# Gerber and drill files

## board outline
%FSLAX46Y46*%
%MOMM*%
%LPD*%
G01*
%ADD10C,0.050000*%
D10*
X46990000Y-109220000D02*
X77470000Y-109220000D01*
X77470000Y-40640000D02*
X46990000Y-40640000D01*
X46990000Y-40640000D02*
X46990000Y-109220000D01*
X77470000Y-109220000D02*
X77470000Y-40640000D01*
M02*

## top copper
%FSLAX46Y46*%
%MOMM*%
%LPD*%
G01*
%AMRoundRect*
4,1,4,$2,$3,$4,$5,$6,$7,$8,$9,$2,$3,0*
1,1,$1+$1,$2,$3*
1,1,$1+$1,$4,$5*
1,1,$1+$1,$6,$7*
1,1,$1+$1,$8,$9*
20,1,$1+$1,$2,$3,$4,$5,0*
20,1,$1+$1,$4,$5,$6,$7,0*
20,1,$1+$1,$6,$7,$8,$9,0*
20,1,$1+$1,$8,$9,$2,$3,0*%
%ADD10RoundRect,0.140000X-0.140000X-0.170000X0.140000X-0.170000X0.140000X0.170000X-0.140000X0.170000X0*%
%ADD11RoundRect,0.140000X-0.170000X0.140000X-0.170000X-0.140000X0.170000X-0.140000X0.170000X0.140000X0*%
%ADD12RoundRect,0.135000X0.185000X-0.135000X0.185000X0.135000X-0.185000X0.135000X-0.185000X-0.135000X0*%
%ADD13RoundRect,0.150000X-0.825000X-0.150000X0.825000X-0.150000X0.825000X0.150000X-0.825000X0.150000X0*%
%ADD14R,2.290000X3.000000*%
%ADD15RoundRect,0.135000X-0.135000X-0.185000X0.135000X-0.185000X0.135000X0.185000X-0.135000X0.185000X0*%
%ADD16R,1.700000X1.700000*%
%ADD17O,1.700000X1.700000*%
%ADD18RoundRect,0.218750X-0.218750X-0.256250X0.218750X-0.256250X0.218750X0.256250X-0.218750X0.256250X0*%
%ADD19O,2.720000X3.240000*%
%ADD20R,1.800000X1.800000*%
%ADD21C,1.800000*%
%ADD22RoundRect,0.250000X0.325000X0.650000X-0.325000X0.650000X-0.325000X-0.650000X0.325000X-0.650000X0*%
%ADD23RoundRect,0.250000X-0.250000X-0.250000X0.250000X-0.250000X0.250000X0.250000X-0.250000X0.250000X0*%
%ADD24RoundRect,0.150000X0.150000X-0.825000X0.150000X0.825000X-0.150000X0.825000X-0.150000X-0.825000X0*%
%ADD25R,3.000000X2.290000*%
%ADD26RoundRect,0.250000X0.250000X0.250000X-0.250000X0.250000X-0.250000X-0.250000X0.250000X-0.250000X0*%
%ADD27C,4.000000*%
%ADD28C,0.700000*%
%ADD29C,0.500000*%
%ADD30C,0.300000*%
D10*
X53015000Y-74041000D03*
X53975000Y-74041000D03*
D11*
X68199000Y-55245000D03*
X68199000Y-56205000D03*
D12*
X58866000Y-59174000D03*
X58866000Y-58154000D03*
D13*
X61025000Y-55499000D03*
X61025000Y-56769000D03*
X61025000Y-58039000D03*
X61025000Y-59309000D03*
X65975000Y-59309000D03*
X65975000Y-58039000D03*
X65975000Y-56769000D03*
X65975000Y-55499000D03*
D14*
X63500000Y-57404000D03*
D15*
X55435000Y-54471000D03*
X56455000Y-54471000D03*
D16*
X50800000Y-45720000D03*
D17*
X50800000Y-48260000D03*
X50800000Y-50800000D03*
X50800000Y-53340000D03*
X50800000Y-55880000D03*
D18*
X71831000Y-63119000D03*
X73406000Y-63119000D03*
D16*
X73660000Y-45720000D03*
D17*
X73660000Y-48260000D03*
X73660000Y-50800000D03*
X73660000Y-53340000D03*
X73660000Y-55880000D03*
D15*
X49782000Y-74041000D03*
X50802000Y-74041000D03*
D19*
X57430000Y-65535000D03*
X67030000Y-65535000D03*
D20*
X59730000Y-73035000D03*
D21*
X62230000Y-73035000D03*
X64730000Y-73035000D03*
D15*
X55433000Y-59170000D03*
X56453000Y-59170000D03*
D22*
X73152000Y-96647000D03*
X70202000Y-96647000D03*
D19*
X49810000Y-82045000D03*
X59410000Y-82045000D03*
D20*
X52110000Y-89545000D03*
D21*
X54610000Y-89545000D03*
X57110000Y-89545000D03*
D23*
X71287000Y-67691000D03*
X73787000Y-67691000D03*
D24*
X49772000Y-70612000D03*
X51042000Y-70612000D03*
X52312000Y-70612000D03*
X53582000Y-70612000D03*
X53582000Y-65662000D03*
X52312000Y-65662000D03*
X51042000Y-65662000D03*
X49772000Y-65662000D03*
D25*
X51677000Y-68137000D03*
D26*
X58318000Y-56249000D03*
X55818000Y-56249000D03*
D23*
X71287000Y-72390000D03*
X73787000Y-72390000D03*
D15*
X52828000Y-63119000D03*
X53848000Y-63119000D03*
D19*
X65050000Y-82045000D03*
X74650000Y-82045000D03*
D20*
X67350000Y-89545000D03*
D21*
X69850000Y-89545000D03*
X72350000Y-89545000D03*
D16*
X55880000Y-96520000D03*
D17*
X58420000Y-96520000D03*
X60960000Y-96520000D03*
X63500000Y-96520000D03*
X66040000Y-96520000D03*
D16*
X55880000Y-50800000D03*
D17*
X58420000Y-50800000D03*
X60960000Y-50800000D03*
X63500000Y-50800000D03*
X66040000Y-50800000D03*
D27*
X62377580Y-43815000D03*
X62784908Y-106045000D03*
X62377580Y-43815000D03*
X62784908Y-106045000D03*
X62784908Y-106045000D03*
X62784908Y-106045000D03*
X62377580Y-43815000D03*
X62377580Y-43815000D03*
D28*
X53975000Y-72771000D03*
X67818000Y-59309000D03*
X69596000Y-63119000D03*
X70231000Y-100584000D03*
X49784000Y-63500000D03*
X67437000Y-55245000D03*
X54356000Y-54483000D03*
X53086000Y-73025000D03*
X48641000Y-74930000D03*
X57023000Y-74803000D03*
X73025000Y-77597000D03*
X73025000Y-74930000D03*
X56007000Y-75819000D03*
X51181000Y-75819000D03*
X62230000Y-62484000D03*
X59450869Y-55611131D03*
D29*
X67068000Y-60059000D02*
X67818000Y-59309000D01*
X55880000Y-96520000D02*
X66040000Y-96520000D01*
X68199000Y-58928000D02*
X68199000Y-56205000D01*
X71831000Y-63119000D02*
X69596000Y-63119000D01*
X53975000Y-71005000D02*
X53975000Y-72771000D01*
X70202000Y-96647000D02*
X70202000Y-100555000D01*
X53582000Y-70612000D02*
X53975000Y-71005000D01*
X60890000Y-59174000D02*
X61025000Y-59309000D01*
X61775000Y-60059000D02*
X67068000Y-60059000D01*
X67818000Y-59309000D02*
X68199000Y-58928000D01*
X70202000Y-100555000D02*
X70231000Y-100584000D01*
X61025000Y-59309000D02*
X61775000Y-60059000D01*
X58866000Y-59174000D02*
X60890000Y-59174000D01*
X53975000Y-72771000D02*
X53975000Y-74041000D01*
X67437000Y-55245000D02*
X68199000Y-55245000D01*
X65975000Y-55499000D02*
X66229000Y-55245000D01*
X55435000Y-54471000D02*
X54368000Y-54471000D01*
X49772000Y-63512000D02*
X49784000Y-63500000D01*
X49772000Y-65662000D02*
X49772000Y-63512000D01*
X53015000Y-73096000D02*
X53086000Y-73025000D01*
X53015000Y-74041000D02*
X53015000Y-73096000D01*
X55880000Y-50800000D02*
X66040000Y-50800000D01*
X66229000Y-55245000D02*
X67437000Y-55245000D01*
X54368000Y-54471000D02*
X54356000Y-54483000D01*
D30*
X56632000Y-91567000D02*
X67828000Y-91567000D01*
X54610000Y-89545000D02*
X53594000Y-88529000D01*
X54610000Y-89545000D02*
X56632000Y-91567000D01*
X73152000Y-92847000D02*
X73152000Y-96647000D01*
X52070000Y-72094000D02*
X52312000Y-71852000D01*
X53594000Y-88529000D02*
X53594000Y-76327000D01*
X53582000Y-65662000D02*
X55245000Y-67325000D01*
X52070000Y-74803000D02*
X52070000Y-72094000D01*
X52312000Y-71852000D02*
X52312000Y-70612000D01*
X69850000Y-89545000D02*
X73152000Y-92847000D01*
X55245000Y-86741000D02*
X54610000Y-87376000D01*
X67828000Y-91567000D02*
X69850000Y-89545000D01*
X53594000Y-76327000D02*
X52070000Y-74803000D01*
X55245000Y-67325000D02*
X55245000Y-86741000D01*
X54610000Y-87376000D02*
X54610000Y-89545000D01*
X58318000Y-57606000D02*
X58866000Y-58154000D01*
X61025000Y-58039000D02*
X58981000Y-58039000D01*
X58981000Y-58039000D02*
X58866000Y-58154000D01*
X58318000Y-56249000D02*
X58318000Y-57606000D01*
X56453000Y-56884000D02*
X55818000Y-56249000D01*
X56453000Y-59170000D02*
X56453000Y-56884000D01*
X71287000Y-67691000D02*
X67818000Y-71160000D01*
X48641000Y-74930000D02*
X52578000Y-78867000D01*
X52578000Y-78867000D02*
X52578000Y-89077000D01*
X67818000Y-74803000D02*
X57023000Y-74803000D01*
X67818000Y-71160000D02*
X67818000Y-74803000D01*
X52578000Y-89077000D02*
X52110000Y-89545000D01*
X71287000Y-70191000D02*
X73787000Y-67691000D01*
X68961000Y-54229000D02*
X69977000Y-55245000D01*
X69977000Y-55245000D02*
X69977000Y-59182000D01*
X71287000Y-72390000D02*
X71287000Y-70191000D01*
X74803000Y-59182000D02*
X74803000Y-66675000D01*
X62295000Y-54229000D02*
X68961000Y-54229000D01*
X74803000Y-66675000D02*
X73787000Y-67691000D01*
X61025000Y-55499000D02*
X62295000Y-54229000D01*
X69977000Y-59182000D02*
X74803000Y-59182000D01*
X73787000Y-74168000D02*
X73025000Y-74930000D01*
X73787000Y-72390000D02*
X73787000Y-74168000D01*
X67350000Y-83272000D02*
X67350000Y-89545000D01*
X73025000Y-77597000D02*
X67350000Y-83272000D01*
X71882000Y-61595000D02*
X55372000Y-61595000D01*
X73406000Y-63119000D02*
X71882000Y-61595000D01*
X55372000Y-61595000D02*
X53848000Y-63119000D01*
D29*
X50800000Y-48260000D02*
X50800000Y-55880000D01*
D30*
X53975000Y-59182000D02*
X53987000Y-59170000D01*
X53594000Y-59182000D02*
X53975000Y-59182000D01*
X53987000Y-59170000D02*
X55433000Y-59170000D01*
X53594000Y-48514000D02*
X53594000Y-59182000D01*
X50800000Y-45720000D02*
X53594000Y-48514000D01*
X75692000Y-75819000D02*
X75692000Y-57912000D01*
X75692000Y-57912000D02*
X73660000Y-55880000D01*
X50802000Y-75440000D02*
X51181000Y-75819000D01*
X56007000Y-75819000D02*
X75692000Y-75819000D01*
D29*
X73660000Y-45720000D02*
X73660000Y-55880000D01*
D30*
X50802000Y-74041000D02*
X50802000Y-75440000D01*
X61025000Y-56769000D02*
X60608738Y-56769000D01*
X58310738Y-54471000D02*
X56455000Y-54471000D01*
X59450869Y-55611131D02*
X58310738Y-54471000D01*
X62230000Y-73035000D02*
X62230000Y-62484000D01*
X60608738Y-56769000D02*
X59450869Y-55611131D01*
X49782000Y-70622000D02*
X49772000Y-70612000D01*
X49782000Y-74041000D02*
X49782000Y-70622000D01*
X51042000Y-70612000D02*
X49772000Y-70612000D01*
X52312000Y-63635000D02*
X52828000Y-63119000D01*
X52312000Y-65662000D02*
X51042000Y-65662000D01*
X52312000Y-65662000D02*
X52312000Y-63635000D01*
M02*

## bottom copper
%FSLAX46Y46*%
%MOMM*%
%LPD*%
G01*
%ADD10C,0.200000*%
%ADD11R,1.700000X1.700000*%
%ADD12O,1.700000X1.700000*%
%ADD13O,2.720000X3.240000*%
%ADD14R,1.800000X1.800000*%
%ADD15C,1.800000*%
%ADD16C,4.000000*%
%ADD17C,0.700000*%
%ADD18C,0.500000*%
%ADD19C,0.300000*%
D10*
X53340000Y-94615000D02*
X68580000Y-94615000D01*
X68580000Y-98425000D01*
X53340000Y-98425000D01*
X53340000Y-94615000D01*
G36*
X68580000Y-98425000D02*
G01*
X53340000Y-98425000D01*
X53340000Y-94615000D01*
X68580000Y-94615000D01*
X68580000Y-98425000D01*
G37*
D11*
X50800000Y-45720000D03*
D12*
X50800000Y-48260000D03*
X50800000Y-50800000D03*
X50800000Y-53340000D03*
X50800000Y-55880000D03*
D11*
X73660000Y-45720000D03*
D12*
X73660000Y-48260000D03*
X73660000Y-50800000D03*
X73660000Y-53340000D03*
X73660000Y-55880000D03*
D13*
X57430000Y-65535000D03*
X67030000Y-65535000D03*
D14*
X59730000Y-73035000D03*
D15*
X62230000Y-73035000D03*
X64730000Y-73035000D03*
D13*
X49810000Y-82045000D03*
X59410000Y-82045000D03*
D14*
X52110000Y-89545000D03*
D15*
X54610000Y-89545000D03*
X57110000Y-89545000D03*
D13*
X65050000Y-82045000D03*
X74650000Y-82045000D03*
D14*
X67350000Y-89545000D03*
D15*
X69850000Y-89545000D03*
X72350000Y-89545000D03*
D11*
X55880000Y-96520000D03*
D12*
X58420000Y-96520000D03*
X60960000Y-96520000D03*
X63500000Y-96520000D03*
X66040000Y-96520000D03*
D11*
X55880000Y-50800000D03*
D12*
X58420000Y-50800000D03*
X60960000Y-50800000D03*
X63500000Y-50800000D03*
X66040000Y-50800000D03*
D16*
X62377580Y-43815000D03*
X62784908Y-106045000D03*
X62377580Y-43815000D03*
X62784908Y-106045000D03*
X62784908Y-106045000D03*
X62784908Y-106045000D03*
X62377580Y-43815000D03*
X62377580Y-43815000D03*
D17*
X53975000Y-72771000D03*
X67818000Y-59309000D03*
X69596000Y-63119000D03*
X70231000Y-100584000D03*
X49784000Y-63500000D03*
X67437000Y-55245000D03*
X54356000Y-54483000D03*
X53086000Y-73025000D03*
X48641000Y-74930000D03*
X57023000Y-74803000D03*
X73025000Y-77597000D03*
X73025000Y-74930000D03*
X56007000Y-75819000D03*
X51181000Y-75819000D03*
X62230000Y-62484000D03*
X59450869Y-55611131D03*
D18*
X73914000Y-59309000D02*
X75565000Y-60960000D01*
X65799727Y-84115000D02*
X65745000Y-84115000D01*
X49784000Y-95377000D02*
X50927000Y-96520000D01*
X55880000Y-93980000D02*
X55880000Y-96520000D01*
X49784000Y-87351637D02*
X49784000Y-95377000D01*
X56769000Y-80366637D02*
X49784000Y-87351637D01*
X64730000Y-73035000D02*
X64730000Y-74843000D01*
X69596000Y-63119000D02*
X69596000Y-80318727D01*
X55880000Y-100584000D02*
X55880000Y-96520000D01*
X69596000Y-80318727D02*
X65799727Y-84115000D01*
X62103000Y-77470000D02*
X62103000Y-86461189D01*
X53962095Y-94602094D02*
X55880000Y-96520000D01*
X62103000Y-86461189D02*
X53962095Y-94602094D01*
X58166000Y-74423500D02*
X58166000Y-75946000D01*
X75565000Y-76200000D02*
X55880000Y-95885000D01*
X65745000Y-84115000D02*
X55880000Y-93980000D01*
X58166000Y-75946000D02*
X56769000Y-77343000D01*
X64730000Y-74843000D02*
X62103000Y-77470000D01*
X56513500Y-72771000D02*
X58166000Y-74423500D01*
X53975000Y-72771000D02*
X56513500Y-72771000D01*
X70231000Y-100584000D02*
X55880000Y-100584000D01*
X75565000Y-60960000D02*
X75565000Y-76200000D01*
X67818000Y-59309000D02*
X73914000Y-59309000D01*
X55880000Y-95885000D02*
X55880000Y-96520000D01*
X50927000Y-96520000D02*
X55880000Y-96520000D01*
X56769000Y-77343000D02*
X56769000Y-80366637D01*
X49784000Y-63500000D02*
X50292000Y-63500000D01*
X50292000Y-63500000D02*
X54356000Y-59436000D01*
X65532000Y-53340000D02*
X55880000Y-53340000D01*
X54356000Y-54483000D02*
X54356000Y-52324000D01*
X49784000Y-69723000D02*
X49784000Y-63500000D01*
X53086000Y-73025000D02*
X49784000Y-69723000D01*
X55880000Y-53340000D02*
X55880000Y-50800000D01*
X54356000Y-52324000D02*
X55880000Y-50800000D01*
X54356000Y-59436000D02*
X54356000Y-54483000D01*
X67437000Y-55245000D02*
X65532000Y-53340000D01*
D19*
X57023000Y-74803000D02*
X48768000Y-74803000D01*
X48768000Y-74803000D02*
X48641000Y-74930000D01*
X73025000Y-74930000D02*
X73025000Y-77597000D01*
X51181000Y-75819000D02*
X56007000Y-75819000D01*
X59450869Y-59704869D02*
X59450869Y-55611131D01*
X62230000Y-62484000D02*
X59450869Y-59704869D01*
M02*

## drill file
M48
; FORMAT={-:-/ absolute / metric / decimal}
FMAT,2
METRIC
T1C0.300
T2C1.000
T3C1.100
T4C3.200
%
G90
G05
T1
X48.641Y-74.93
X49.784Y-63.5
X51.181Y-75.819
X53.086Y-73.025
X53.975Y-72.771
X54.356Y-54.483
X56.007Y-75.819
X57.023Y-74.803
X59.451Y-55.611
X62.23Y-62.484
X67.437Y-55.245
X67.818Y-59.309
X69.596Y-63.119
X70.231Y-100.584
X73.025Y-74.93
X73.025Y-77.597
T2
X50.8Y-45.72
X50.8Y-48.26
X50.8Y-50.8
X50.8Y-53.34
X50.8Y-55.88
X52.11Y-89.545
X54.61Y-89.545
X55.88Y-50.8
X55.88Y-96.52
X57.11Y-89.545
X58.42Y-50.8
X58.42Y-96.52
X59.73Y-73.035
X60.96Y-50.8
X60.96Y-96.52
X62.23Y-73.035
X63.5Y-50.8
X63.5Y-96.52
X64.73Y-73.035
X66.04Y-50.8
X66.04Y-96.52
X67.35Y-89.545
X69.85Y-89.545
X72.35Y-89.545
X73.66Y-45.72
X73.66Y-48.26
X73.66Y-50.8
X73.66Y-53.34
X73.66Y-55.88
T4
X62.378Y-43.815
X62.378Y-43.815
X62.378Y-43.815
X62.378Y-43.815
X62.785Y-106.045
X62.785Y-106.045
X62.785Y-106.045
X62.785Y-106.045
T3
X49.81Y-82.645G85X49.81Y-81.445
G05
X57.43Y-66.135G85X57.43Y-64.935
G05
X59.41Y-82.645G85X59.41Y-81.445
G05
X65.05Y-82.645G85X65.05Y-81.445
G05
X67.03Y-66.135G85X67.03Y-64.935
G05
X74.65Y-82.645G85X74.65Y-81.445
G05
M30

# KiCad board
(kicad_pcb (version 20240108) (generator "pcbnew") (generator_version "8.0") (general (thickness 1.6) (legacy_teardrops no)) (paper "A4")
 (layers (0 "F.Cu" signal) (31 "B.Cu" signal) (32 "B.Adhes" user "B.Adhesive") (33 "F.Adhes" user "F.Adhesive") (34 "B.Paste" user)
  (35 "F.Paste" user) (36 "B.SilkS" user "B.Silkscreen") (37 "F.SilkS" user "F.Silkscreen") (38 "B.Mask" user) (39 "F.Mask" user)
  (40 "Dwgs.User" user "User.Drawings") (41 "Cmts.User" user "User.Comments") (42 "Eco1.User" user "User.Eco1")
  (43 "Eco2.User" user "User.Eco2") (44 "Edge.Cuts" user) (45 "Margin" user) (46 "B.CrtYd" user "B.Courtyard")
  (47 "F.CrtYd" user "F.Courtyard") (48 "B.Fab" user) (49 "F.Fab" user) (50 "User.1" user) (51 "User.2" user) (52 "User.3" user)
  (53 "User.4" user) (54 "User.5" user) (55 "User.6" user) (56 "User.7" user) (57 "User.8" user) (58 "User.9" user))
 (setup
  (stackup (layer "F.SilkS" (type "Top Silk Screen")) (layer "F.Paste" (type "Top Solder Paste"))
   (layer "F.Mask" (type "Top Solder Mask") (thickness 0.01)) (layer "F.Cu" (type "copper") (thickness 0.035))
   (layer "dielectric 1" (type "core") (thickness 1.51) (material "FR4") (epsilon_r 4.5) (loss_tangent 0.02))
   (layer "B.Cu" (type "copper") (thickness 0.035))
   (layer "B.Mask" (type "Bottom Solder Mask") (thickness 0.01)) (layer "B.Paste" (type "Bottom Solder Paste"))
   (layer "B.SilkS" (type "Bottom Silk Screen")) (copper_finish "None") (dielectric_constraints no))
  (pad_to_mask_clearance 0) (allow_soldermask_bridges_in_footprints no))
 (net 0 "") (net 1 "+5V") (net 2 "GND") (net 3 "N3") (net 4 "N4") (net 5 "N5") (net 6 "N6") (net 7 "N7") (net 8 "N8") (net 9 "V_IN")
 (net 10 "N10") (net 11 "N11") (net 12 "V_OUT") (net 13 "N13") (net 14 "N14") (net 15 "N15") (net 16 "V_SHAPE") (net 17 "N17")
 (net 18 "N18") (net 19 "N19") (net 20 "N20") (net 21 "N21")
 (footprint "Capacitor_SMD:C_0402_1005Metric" (layer "F.Cu") (at 53.495 74.041)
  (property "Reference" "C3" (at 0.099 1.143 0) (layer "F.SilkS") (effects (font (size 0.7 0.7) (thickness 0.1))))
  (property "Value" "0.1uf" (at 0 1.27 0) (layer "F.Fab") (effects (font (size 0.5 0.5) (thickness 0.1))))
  (pad "1" smd roundrect (at -0.48 0) (size 0.56 0.62) (layers "F.Cu" "F.Paste" "F.Mask") (roundrect_rratio 0.25) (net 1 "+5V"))
  (pad "2" smd roundrect (at 0.48 0) (size 0.56 0.62) (layers "F.Cu" "F.Paste" "F.Mask") (roundrect_rratio 0.25) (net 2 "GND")))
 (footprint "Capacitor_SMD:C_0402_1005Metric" (layer "F.Cu") (at 68.199 55.725 -90)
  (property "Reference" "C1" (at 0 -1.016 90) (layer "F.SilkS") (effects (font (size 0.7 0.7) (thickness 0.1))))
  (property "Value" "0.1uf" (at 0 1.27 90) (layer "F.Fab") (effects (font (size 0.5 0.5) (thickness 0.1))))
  (pad "1" smd roundrect (at -0.48 0 270) (size 0.56 0.62) (layers "F.Cu" "F.Paste" "F.Mask") (roundrect_rratio 0.25) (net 1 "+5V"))
  (pad "2" smd roundrect (at 0.48 0 270) (size 0.56 0.62) (layers "F.Cu" "F.Paste" "F.Mask") (roundrect_rratio 0.25) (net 2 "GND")))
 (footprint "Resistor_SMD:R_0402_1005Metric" (layer "F.Cu") (at 58.866 58.664 90)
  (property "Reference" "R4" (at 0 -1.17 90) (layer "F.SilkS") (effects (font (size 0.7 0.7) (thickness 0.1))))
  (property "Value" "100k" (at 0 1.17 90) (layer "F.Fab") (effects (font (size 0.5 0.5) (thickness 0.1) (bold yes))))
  (pad "1" smd roundrect (at -0.51 0 90) (size 0.54 0.64) (layers "F.Cu" "F.Paste" "F.Mask") (roundrect_rratio 0.25) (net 2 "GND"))
  (pad "2" smd roundrect (at 0.51 0 90) (size 0.54 0.64) (layers "F.Cu" "F.Paste" "F.Mask") (roundrect_rratio 0.25) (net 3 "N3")))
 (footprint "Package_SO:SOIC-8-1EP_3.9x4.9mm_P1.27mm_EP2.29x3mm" (layer "F.Cu") (at 63.5 57.404)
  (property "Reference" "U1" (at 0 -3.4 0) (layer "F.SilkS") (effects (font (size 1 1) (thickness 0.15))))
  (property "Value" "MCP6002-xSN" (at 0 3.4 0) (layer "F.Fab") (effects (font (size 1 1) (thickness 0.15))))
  (pad "" smd roundrect (at -0.57 -0.75) (size 0.92 1.21) (layers "F.Paste") (roundrect_rratio 0.25))
  (pad "" smd roundrect (at -0.57 0.75) (size 0.92 1.21) (layers "F.Paste") (roundrect_rratio 0.25))
  (pad "" smd roundrect (at 0.57 -0.75) (size 0.92 1.21) (layers "F.Paste") (roundrect_rratio 0.25))
  (pad "" smd roundrect (at 0.57 0.75) (size 0.92 1.21) (layers "F.Paste") (roundrect_rratio 0.25))
  (pad "1" smd roundrect (at -2.475 -1.905) (size 1.95 0.6) (layers "F.Cu" "F.Paste" "F.Mask") (roundrect_rratio 0.25) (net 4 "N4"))
  (pad "2" smd roundrect (at -2.475 -0.635) (size 1.95 0.6) (layers "F.Cu" "F.Paste" "F.Mask") (roundrect_rratio 0.25) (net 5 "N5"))
  (pad "3" smd roundrect (at -2.475 0.635) (size 1.95 0.6) (layers "F.Cu" "F.Paste" "F.Mask") (roundrect_rratio 0.25) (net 3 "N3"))
  (pad "4" smd roundrect (at -2.475 1.905) (size 1.95 0.6) (layers "F.Cu" "F.Paste" "F.Mask") (roundrect_rratio 0.25) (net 2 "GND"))
  (pad "5" smd roundrect (at 2.475 1.905) (size 1.95 0.6) (layers "F.Cu" "F.Paste" "F.Mask") (roundrect_rratio 0.25) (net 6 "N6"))
  (pad "6" smd roundrect (at 2.475 0.635) (size 1.95 0.6) (layers "F.Cu" "F.Paste" "F.Mask") (roundrect_rratio 0.25) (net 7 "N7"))
  (pad "7" smd roundrect (at 2.475 -0.635) (size 1.95 0.6) (layers "F.Cu" "F.Paste" "F.Mask") (roundrect_rratio 0.25) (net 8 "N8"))
  (pad "8" smd roundrect (at 2.475 -1.905) (size 1.95 0.6) (layers "F.Cu" "F.Paste" "F.Mask") (roundrect_rratio 0.25) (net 1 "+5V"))
  (pad "9" smd rect (at 0 0) (size 2.29 3) (layers "F.Cu" "F.Mask") (zone_connect 2)))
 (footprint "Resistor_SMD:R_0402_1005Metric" (layer "F.Cu") (at 55.945 54.471)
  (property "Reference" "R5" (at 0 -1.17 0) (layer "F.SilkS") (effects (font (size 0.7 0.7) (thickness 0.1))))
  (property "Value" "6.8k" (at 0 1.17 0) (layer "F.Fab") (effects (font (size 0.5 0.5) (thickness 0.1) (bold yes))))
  (pad "1" smd roundrect (at -0.51 0) (size 0.54 0.64) (layers "F.Cu" "F.Paste" "F.Mask") (roundrect_rratio 0.25) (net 1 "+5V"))
  (pad "2" smd roundrect (at 0.51 0) (size 0.54 0.64) (layers "F.Cu" "F.Paste" "F.Mask") (roundrect_rratio 0.25) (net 5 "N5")))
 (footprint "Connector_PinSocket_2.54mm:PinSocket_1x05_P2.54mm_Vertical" (layer "F.Cu") (at 50.8 45.72)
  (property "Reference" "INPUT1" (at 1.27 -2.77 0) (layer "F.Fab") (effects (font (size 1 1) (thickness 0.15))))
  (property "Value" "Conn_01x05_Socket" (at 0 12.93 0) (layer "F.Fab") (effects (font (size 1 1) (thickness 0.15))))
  (pad "1" thru_hole rect (at 0 0) (size 1.7 1.7) (drill 1) (layers "*.Cu" "*.Mask") (remove_unused_layers no) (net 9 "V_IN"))
  (pad "2" thru_hole oval (at 0 2.54) (size 1.7 1.7) (drill 1) (layers "*.Cu" "*.Mask") (remove_unused_layers no) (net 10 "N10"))
  (pad "3" thru_hole oval (at 0 5.08) (size 1.7 1.7) (drill 1) (layers "*.Cu" "*.Mask") (remove_unused_layers no) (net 10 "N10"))
  (pad "4" thru_hole oval (at 0 7.62) (size 1.7 1.7) (drill 1) (layers "*.Cu" "*.Mask") (remove_unused_layers no) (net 10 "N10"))
  (pad "5" thru_hole oval (at 0 10.16) (size 1.7 1.7) (drill 1) (layers "*.Cu" "*.Mask") (remove_unused_layers no) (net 10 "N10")))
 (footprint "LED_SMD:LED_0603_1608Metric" (layer "F.Cu") (at 72.6185 63.119)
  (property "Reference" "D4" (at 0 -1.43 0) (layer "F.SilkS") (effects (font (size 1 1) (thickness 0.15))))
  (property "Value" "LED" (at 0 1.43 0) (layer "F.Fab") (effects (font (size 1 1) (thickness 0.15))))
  (pad "1" smd roundrect (at -0.7875 0) (size 0.875 0.95) (layers "F.Cu" "F.Paste" "F.Mask") (roundrect_rratio 0.25) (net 2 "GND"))
  (pad "2" smd roundrect (at 0.7875 0) (size 0.875 0.95) (layers "F.Cu" "F.Paste" "F.Mask") (roundrect_rratio 0.25) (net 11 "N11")))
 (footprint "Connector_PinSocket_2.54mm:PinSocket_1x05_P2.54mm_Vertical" (layer "F.Cu") (at 73.66 45.72)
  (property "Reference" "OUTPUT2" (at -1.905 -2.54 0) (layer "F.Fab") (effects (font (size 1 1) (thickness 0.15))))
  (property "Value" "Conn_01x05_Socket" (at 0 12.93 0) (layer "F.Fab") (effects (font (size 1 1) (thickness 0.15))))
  (pad "1" thru_hole rect (at 0 0) (size 1.7 1.7) (drill 1) (layers "*.Cu" "*.Mask") (remove_unused_layers no) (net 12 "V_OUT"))
  (pad "2" thru_hole oval (at 0 2.54) (size 1.7 1.7) (drill 1) (layers "*.Cu" "*.Mask") (remove_unused_layers no) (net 12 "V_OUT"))
  (pad "3" thru_hole oval (at 0 5.08) (size 1.7 1.7) (drill 1) (layers "*.Cu" "*.Mask") (remove_unused_layers no) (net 12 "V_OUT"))
  (pad "4" thru_hole oval (at 0 7.62) (size 1.7 1.7) (drill 1) (layers "*.Cu" "*.Mask") (remove_unused_layers no) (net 12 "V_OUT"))
  (pad "5" thru_hole oval (at 0 10.16) (size 1.7 1.7) (drill 1) (layers "*.Cu" "*.Mask") (remove_unused_layers no) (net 12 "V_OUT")))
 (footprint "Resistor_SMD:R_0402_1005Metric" (layer "F.Cu") (at 50.292 74.041)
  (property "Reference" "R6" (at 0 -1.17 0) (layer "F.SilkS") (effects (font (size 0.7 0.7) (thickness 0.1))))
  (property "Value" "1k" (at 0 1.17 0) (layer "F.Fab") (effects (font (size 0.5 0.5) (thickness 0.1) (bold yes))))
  (pad "1" smd roundrect (at -0.51 0) (size 0.54 0.64) (layers "F.Cu" "F.Paste" "F.Mask") (roundrect_rratio 0.25) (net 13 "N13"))
  (pad "2" smd roundrect (at 0.51 0) (size 0.54 0.64) (layers "F.Cu" "F.Paste" "F.Mask") (roundrect_rratio 0.25) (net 12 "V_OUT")))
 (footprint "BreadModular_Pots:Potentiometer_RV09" (layer "F.Cu") (at 59.73 73.035 90)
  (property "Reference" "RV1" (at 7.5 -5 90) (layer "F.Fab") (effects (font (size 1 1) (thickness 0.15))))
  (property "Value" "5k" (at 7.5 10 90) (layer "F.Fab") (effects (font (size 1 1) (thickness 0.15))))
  (pad "" thru_hole oval (at 7.5 -2.3 180) (size 2.72 3.24) (drill oval 1.1 2.3) (layers "*.Cu" "*.Mask") (remove_unused_layers no))
  (pad "" thru_hole oval (at 7.5 7.3 180) (size 2.72 3.24) (drill oval 1.1 2.3) (layers "*.Cu" "*.Mask") (remove_unused_layers no))
  (pad "1" thru_hole rect (at 0 0 180) (size 1.8 1.8) (drill 1) (layers "*.Cu" "*.Mask") (remove_unused_layers no) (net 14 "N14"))
  (pad "2" thru_hole circle (at 0 2.5 180) (size 1.8 1.8) (drill 1) (layers "*.Cu" "*.Mask") (remove_unused_layers no) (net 5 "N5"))
  (pad "3" thru_hole circle (at 0 5 180) (size 1.8 1.8) (drill 1) (layers "*.Cu" "*.Mask") (remove_unused_layers no) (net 2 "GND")))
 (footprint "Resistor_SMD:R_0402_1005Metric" (layer "F.Cu") (at 55.943 59.17)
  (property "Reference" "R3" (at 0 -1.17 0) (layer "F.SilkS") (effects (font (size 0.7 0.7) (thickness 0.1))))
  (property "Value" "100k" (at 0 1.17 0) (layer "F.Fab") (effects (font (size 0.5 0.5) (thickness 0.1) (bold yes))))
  (pad "1" smd roundrect (at -0.51 0) (size 0.54 0.64) (layers "F.Cu" "F.Paste" "F.Mask") (roundrect_rratio 0.25) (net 9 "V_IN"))
  (pad "2" smd roundrect (at 0.51 0) (size 0.54 0.64) (layers "F.Cu" "F.Paste" "F.Mask") (roundrect_rratio 0.25) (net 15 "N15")))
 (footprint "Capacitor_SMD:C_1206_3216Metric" (layer "F.Cu") (at 71.677 96.647 180)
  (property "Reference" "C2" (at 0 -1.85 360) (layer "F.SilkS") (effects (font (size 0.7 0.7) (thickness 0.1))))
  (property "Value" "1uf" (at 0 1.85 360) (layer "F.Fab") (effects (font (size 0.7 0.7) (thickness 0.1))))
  (pad "1" smd roundrect (at -1.475 0 180) (size 1.15 1.8) (layers "F.Cu" "F.Paste" "F.Mask") (roundrect_rratio 0.217391) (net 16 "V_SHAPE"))
  (pad "2" smd roundrect (at 1.475 0 180) (size 1.15 1.8) (layers "F.Cu" "F.Paste" "F.Mask") (roundrect_rratio 0.217391) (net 2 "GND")))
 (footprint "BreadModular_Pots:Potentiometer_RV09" (layer "F.Cu") (at 52.11 89.545 90)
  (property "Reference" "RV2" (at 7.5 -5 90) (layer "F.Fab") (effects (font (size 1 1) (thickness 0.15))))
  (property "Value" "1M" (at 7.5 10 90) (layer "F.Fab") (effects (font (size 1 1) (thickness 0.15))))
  (pad "" thru_hole oval (at 7.5 -2.3 180) (size 2.72 3.24) (drill oval 1.1 2.3) (layers "*.Cu" "*.Mask") (remove_unused_layers no))
  (pad "" thru_hole oval (at 7.5 7.3 180) (size 2.72 3.24) (drill oval 1.1 2.3) (layers "*.Cu" "*.Mask") (remove_unused_layers no))
  (pad "1" thru_hole rect (at 0 0 180) (size 1.8 1.8) (drill 1) (layers "*.Cu" "*.Mask") (remove_unused_layers no) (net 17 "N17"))
  (pad "2" thru_hole circle (at 0 2.5 180) (size 1.8 1.8) (drill 1) (layers "*.Cu" "*.Mask") (remove_unused_layers no) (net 16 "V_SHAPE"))
  (pad "3" thru_hole circle (at 0 5 180) (size 1.8 1.8) (drill 1) (layers "*.Cu" "*.Mask") (remove_unused_layers no) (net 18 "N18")))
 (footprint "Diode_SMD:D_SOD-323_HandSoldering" (layer "F.Cu") (at 72.537 67.691)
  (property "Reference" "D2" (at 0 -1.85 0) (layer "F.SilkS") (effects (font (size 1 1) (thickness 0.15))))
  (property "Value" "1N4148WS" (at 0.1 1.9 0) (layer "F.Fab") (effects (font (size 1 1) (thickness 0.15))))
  (pad "1" smd roundrect (at -1.25 0) (size 1 1) (layers "F.Cu" "F.Paste" "F.Mask") (roundrect_rratio 0.25) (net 17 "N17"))
  (pad "2" smd roundrect (at 1.25 0) (size 1 1) (layers "F.Cu" "F.Paste" "F.Mask") (roundrect_rratio 0.25) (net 4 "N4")))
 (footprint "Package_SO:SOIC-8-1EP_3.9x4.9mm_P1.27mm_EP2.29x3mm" (layer "F.Cu") (at 51.677 68.137 90)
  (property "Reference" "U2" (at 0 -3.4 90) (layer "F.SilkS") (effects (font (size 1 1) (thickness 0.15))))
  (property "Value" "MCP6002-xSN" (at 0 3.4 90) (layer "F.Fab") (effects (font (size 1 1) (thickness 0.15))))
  (pad "" smd roundrect (at -0.57 -0.75 90) (size 0.92 1.21) (layers "F.Paste") (roundrect_rratio 0.25))
  (pad "" smd roundrect (at -0.57 0.75 90) (size 0.92 1.21) (layers "F.Paste") (roundrect_rratio 0.25))
  (pad "" smd roundrect (at 0.57 -0.75 90) (size 0.92 1.21) (layers "F.Paste") (roundrect_rratio 0.25))
  (pad "" smd roundrect (at 0.57 0.75 90) (size 0.92 1.21) (layers "F.Paste") (roundrect_rratio 0.25))
  (pad "1" smd roundrect (at -2.475 -1.905 90) (size 1.95 0.6) (layers "F.Cu" "F.Paste" "F.Mask") (roundrect_rratio 0.25) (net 13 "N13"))
  (pad "2" smd roundrect (at -2.475 -0.635 90) (size 1.95 0.6) (layers "F.Cu" "F.Paste" "F.Mask") (roundrect_rratio 0.25) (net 13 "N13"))
  (pad "3" smd roundrect (at -2.475 0.635 90) (size 1.95 0.6) (layers "F.Cu" "F.Paste" "F.Mask") (roundrect_rratio 0.25) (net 16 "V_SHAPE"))
  (pad "4" smd roundrect (at -2.475 1.905 90) (size 1.95 0.6) (layers "F.Cu" "F.Paste" "F.Mask") (roundrect_rratio 0.25) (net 2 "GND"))
  (pad "5" smd roundrect (at 2.475 1.905 90) (size 1.95 0.6) (layers "F.Cu" "F.Paste" "F.Mask") (roundrect_rratio 0.25) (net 16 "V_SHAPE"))
  (pad "6" smd roundrect (at 2.475 0.635 90) (size 1.95 0.6) (layers "F.Cu" "F.Paste" "F.Mask") (roundrect_rratio 0.25) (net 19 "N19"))
  (pad "7" smd roundrect (at 2.475 -0.635 90) (size 1.95 0.6) (layers "F.Cu" "F.Paste" "F.Mask") (roundrect_rratio 0.25) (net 19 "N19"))
  (pad "8" smd roundrect (at 2.475 -1.905 90) (size 1.95 0.6) (layers "F.Cu" "F.Paste" "F.Mask") (roundrect_rratio 0.25) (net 1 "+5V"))
  (pad "9" smd rect (at 0 0 90) (size 2.29 3) (layers "F.Cu" "F.Mask") (zone_connect 2)))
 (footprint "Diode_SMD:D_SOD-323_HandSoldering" (layer "F.Cu") (at 57.068 56.249 180)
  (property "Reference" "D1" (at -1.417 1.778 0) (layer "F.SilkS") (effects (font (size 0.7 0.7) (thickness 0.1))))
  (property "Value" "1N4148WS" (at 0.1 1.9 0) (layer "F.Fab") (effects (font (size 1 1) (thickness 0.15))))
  (pad "1" smd roundrect (at -1.25 0 180) (size 1 1) (layers "F.Cu" "F.Paste" "F.Mask") (roundrect_rratio 0.25) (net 3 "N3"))
  (pad "2" smd roundrect (at 1.25 0 180) (size 1 1) (layers "F.Cu" "F.Paste" "F.Mask") (roundrect_rratio 0.25) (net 15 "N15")))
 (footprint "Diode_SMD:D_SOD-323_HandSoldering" (layer "F.Cu") (at 72.537 72.39)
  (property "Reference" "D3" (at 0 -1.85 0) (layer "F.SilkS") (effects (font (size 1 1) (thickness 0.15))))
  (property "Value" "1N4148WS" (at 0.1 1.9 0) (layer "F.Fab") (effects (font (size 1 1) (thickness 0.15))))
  (pad "1" smd roundrect (at -1.25 0) (size 1 1) (layers "F.Cu" "F.Paste" "F.Mask") (roundrect_rratio 0.25) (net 4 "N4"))
  (pad "2" smd roundrect (at 1.25 0) (size 1 1) (layers "F.Cu" "F.Paste" "F.Mask") (roundrect_rratio 0.25) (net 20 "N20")))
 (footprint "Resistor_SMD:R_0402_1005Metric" (layer "F.Cu") (at 53.338 63.119)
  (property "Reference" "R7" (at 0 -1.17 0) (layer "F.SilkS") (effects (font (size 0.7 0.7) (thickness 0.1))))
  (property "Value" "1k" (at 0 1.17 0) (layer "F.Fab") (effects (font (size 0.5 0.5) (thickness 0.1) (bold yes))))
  (pad "1" smd roundrect (at -0.51 0) (size 0.54 0.64) (layers "F.Cu" "F.Paste" "F.Mask") (roundrect_rratio 0.25) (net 19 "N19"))
  (pad "2" smd roundrect (at 0.51 0) (size 0.54 0.64) (layers "F.Cu" "F.Paste" "F.Mask") (roundrect_rratio 0.25) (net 11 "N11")))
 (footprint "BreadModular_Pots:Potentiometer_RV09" (layer "F.Cu") (at 67.35 89.545 90)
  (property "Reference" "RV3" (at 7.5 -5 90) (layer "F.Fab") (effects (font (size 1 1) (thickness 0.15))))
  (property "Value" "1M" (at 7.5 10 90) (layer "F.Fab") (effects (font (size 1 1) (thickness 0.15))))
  (pad "" thru_hole oval (at 7.5 -2.3 180) (size 2.72 3.24) (drill oval 1.1 2.3) (layers "*.Cu" "*.Mask") (remove_unused_layers no))
  (pad "" thru_hole oval (at 7.5 7.3 180) (size 2.72 3.24) (drill oval 1.1 2.3) (layers "*.Cu" "*.Mask") (remove_unused_layers no))
  (pad "1" thru_hole rect (at 0 0 180) (size 1.8 1.8) (drill 1) (layers "*.Cu" "*.Mask") (remove_unused_layers no) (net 20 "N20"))
  (pad "2" thru_hole circle (at 0 2.5 180) (size 1.8 1.8) (drill 1) (layers "*.Cu" "*.Mask") (remove_unused_layers no) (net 16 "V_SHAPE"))
  (pad "3" thru_hole circle (at 0 5 180) (size 1.8 1.8) (drill 1) (layers "*.Cu" "*.Mask") (remove_unused_layers no) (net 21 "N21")))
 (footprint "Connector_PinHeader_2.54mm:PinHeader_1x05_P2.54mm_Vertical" (layer "B.Cu") (at 55.88 96.52 -90)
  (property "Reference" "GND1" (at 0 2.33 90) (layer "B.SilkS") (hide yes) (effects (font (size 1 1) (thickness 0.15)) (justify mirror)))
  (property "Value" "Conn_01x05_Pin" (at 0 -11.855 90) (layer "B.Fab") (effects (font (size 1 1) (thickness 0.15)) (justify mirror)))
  (pad "1" thru_hole rect (at 0 0 270) (size 1.7 1.7) (drill 1) (layers "*.Cu" "*.Mask") (remove_unused_layers no) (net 2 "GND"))
  (pad "2" thru_hole oval (at 0 -2.54 270) (size 1.7 1.7) (drill 1) (layers "*.Cu" "*.Mask") (remove_unused_layers no) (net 2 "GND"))
  (pad "3" thru_hole oval (at 0 -5.08 270) (size 1.7 1.7) (drill 1) (layers "*.Cu" "*.Mask") (remove_unused_layers no) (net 2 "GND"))
  (pad "4" thru_hole oval (at 0 -7.62 270) (size 1.7 1.7) (drill 1) (layers "*.Cu" "*.Mask") (remove_unused_layers no) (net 2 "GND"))
  (pad "5" thru_hole oval (at 0 -10.16 270) (size 1.7 1.7) (drill 1) (layers "*.Cu" "*.Mask") (remove_unused_layers no) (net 2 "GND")))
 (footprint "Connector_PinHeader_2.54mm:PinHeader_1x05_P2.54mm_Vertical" (layer "B.Cu") (at 55.88 50.8 -90)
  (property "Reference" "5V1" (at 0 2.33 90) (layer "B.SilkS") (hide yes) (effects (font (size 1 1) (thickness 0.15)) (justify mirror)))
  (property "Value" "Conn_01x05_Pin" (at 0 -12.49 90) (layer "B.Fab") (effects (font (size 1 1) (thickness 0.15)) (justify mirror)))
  (pad "1" thru_hole rect (at 0 0 270) (size 1.7 1.7) (drill 1) (layers "*.Cu" "*.Mask") (remove_unused_layers no) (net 1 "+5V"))
  (pad "2" thru_hole oval (at 0 -2.54 270) (size 1.7 1.7) (drill 1) (layers "*.Cu" "*.Mask") (remove_unused_layers no) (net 1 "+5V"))
  (pad "3" thru_hole oval (at 0 -5.08 270) (size 1.7 1.7) (drill 1) (layers "*.Cu" "*.Mask") (remove_unused_layers no) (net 1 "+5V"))
  (pad "4" thru_hole oval (at 0 -7.62 270) (size 1.7 1.7) (drill 1) (layers "*.Cu" "*.Mask") (remove_unused_layers no) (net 1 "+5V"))
  (pad "5" thru_hole oval (at 0 -10.16 270) (size 1.7 1.7) (drill 1) (layers "*.Cu" "*.Mask") (remove_unused_layers no) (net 1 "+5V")))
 (gr_poly
  (pts (xy 53.34 94.615) (xy 68.58 94.615) (xy 68.58 98.425) (xy 53.34 98.425)) (stroke (width 0.2) (type solid)) (fill solid)
  (layer "B.Cu") (net 2))
 (gr_line (start 46.99 109.22) (end 77.47 109.22) (stroke (width 0.05) (type default)) (layer "Edge.Cuts"))
 (gr_line (start 77.47 40.64) (end 46.99 40.64) (stroke (width 0.05) (type default)) (layer "Edge.Cuts"))
 (gr_line (start 46.99 40.64) (end 46.99 109.22) (stroke (width 0.05) (type default)) (layer "Edge.Cuts"))
 (gr_line (start 77.47 109.22) (end 77.47 40.64) (stroke (width 0.05) (type default)) (layer "Edge.Cuts"))
 (via (at 62.37758 43.815) (size 4) (drill 3.2) (layers "F.Cu" "B.Cu") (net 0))
 (via (at 62.784908 106.045) (size 4) (drill 3.2) (layers "F.Cu" "B.Cu") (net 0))
 (via (at 62.37758 43.815) (size 4) (drill 3.2) (layers "F.Cu" "B.Cu") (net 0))
 (via (at 62.784908 106.045) (size 4) (drill 3.2) (layers "F.Cu" "B.Cu") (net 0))
 (via (at 62.784908 106.045) (size 4) (drill 3.2) (layers "F.Cu" "B.Cu") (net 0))
 (via (at 62.784908 106.045) (size 4) (drill 3.2) (layers "F.Cu" "B.Cu") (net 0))
 (via (at 62.37758 43.815) (size 4) (drill 3.2) (layers "F.Cu" "B.Cu") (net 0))
 (via (at 62.37758 43.815) (size 4) (drill 3.2) (layers "F.Cu" "B.Cu") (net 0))
 (segment (start 67.068 60.059) (end 67.818 59.309) (width 0.5) (layer "F.Cu") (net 2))
 (segment (start 55.88 96.52) (end 66.04 96.52) (width 0.5) (layer "F.Cu") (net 2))
 (segment (start 68.199 58.928) (end 68.199 56.205) (width 0.5) (layer "F.Cu") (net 2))
 (segment (start 71.831 63.119) (end 69.596 63.119) (width 0.5) (layer "F.Cu") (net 2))
 (segment (start 53.975 71.005) (end 53.975 72.771) (width 0.5) (layer "F.Cu") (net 2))
 (segment (start 70.202 96.647) (end 70.202 100.555) (width 0.5) (layer "F.Cu") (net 2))
 (segment (start 53.582 70.612) (end 53.975 71.005) (width 0.5) (layer "F.Cu") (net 2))
 (segment (start 60.89 59.174) (end 61.025 59.309) (width 0.5) (layer "F.Cu") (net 2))
 (segment (start 61.775 60.059) (end 67.068 60.059) (width 0.5) (layer "F.Cu") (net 2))
 (segment (start 67.818 59.309) (end 68.199 58.928) (width 0.5) (layer "F.Cu") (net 2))
 (segment (start 70.202 100.555) (end 70.231 100.584) (width 0.5) (layer "F.Cu") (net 2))
 (segment (start 61.025 59.309) (end 61.775 60.059) (width 0.5) (layer "F.Cu") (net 2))
 (segment (start 58.866 59.174) (end 60.89 59.174) (width 0.5) (layer "F.Cu") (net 2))
 (segment (start 53.975 72.771) (end 53.975 74.041) (width 0.5) (layer "F.Cu") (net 2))
 (via (at 53.975 72.771) (size 0.7) (drill 0.3) (layers "F.Cu" "B.Cu") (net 2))
 (via (at 67.818 59.309) (size 0.7) (drill 0.3) (layers "F.Cu" "B.Cu") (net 2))
 (via (at 69.596 63.119) (size 0.7) (drill 0.3) (layers "F.Cu" "B.Cu") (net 2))
 (via (at 70.231 100.584) (size 0.7) (drill 0.3) (layers "F.Cu" "B.Cu") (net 2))
 (segment (start 73.914 59.309) (end 75.565 60.96) (width 0.5) (layer "B.Cu") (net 2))
 (segment (start 65.799727 84.115) (end 65.745 84.115) (width 0.5) (layer "B.Cu") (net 2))
 (segment (start 49.784 95.377) (end 50.927 96.52) (width 0.5) (layer "B.Cu") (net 2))
 (segment (start 55.88 93.98) (end 55.88 96.52) (width 0.5) (layer "B.Cu") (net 2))
 (segment (start 49.784 87.351637) (end 49.784 95.377) (width 0.5) (layer "B.Cu") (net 2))
 (segment (start 56.769 80.366637) (end 49.784 87.351637) (width 0.5) (layer "B.Cu") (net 2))
 (segment (start 64.73 73.035) (end 64.73 74.843) (width 0.5) (layer "B.Cu") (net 2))
 (segment (start 69.596 63.119) (end 69.596 80.318727) (width 0.5) (layer "B.Cu") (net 2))
 (segment (start 55.88 100.584) (end 55.88 96.52) (width 0.5) (layer "B.Cu") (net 2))
 (segment (start 69.596 80.318727) (end 65.799727 84.115) (width 0.5) (layer "B.Cu") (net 2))
 (segment (start 62.103 77.47) (end 62.103 86.461189) (width 0.5) (layer "B.Cu") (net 2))
 (segment (start 53.962095 94.602094) (end 55.88 96.52) (width 0.5) (layer "B.Cu") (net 2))
 (segment (start 62.103 86.461189) (end 53.962095 94.602094) (width 0.5) (layer "B.Cu") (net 2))
 (segment (start 58.166 74.4235) (end 58.166 75.946) (width 0.5) (layer "B.Cu") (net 2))
 (segment (start 75.565 76.2) (end 55.88 95.885) (width 0.5) (layer "B.Cu") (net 2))
 (segment (start 65.745 84.115) (end 55.88 93.98) (width 0.5) (layer "B.Cu") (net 2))
 (segment (start 58.166 75.946) (end 56.769 77.343) (width 0.5) (layer "B.Cu") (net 2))
 (segment (start 64.73 74.843) (end 62.103 77.47) (width 0.5) (layer "B.Cu") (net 2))
 (segment (start 56.5135 72.771) (end 58.166 74.4235) (width 0.5) (layer "B.Cu") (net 2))
 (segment (start 53.975 72.771) (end 56.5135 72.771) (width 0.5) (layer "B.Cu") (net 2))
 (segment (start 70.231 100.584) (end 55.88 100.584) (width 0.5) (layer "B.Cu") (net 2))
 (segment (start 75.565 60.96) (end 75.565 76.2) (width 0.5) (layer "B.Cu") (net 2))
 (segment (start 67.818 59.309) (end 73.914 59.309) (width 0.5) (layer "B.Cu") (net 2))
 (segment (start 55.88 95.885) (end 55.88 96.52) (width 0.5) (layer "B.Cu") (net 2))
 (segment (start 50.927 96.52) (end 55.88 96.52) (width 0.5) (layer "B.Cu") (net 2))
 (segment (start 56.769 77.343) (end 56.769 80.366637) (width 0.5) (layer "B.Cu") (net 2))
 (segment (start 67.437 55.245) (end 68.199 55.245) (width 0.5) (layer "F.Cu") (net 1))
 (segment (start 65.975 55.499) (end 66.229 55.245) (width 0.5) (layer "F.Cu") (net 1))
 (segment (start 55.435 54.471) (end 54.368 54.471) (width 0.5) (layer "F.Cu") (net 1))
 (segment (start 49.772 63.512) (end 49.784 63.5) (width 0.5) (layer "F.Cu") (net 1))
 (segment (start 49.772 65.662) (end 49.772 63.512) (width 0.5) (layer "F.Cu") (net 1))
 (segment (start 53.015 73.096) (end 53.086 73.025) (width 0.5) (layer "F.Cu") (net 1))
 (segment (start 53.015 74.041) (end 53.015 73.096) (width 0.5) (layer "F.Cu") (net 1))
 (segment (start 55.88 50.8) (end 66.04 50.8) (width 0.5) (layer "F.Cu") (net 1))
 (segment (start 66.229 55.245) (end 67.437 55.245) (width 0.5) (layer "F.Cu") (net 1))
 (segment (start 54.368 54.471) (end 54.356 54.483) (width 0.5) (layer "F.Cu") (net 1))
 (via (at 49.784 63.5) (size 0.7) (drill 0.3) (layers "F.Cu" "B.Cu") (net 1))
 (via (at 67.437 55.245) (size 0.7) (drill 0.3) (layers "F.Cu" "B.Cu") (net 1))
 (via (at 54.356 54.483) (size 0.7) (drill 0.3) (layers "F.Cu" "B.Cu") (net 1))
 (via (at 53.086 73.025) (size 0.7) (drill 0.3) (layers "F.Cu" "B.Cu") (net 1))
 (segment (start 49.784 63.5) (end 50.292 63.5) (width 0.5) (layer "B.Cu") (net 1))
 (segment (start 50.292 63.5) (end 54.356 59.436) (width 0.5) (layer "B.Cu") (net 1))
 (segment (start 65.532 53.34) (end 55.88 53.34) (width 0.5) (layer "B.Cu") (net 1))
 (segment (start 54.356 54.483) (end 54.356 52.324) (width 0.5) (layer "B.Cu") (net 1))
 (segment (start 49.784 69.723) (end 49.784 63.5) (width 0.5) (layer "B.Cu") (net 1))
 (segment (start 53.086 73.025) (end 49.784 69.723) (width 0.5) (layer "B.Cu") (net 1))
 (segment (start 55.88 53.34) (end 55.88 50.8) (width 0.5) (layer "B.Cu") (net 1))
 (segment (start 54.356 52.324) (end 55.88 50.8) (width 0.5) (layer "B.Cu") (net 1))
 (segment (start 54.356 59.436) (end 54.356 54.483) (width 0.5) (layer "B.Cu") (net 1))
 (segment (start 67.437 55.245) (end 65.532 53.34) (width 0.5) (layer "B.Cu") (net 1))
 (segment (start 56.632 91.567) (end 67.828 91.567) (width 0.3) (layer "F.Cu") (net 16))
 (segment (start 54.61 89.545) (end 53.594 88.529) (width 0.3) (layer "F.Cu") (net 16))
 (segment (start 54.61 89.545) (end 56.632 91.567) (width 0.3) (layer "F.Cu") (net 16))
 (segment (start 73.152 92.847) (end 73.152 96.647) (width 0.3) (layer "F.Cu") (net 16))
 (segment (start 52.07 72.094) (end 52.312 71.852) (width 0.3) (layer "F.Cu") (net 16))
 (segment (start 53.594 88.529) (end 53.594 76.327) (width 0.3) (layer "F.Cu") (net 16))
 (segment (start 53.582 65.662) (end 55.245 67.325) (width 0.3) (layer "F.Cu") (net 16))
 (segment (start 52.07 74.803) (end 52.07 72.094) (width 0.3) (layer "F.Cu") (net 16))
 (segment (start 52.312 71.852) (end 52.312 70.612) (width 0.3) (layer "F.Cu") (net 16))
 (segment (start 69.85 89.545) (end 73.152 92.847) (width 0.3) (layer "F.Cu") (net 16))
 (segment (start 55.245 86.741) (end 54.61 87.376) (width 0.3) (layer "F.Cu") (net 16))
 (segment (start 67.828 91.567) (end 69.85 89.545) (width 0.3) (layer "F.Cu") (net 16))
 (segment (start 53.594 76.327) (end 52.07 74.803) (width 0.3) (layer "F.Cu") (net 16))
 (segment (start 55.245 67.325) (end 55.245 86.741) (width 0.3) (layer "F.Cu") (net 16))
 (segment (start 54.61 87.376) (end 54.61 89.545) (width 0.3) (layer "F.Cu") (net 16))
 (segment (start 58.318 57.606) (end 58.866 58.154) (width 0.3) (layer "F.Cu") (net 3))
 (segment (start 61.025 58.039) (end 58.981 58.039) (width 0.3) (layer "F.Cu") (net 3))
 (segment (start 58.981 58.039) (end 58.866 58.154) (width 0.3) (layer "F.Cu") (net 3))
 (segment (start 58.318 56.249) (end 58.318 57.606) (width 0.3) (layer "F.Cu") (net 3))
 (segment (start 56.453 56.884) (end 55.818 56.249) (width 0.3) (layer "F.Cu") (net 15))
 (segment (start 56.453 59.17) (end 56.453 56.884) (width 0.3) (layer "F.Cu") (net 15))
 (segment (start 71.287 67.691) (end 67.818 71.16) (width 0.3) (layer "F.Cu") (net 17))
 (segment (start 48.641 74.93) (end 52.578 78.867) (width 0.3) (layer "F.Cu") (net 17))
 (segment (start 52.578 78.867) (end 52.578 89.077) (width 0.3) (layer "F.Cu") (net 17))
 (segment (start 67.818 74.803) (end 57.023 74.803) (width 0.3) (layer "F.Cu") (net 17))
 (segment (start 67.818 71.16) (end 67.818 74.803) (width 0.3) (layer "F.Cu") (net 17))
 (segment (start 52.578 89.077) (end 52.11 89.545) (width 0.3) (layer "F.Cu") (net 17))
 (via (at 48.641 74.93) (size 0.7) (drill 0.3) (layers "F.Cu" "B.Cu") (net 17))
 (via (at 57.023 74.803) (size 0.7) (drill 0.3) (layers "F.Cu" "B.Cu") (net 17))
 (segment (start 57.023 74.803) (end 48.768 74.803) (width 0.3) (layer "B.Cu") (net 17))
 (segment (start 48.768 74.803) (end 48.641 74.93) (width 0.3) (layer "B.Cu") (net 17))
 (segment (start 71.287 70.191) (end 73.787 67.691) (width 0.3) (layer "F.Cu") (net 4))
 (segment (start 68.961 54.229) (end 69.977 55.245) (width 0.3) (layer "F.Cu") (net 4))
 (segment (start 69.977 55.245) (end 69.977 59.182) (width 0.3) (layer "F.Cu") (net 4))
 (segment (start 71.287 72.39) (end 71.287 70.191) (width 0.3) (layer "F.Cu") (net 4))
 (segment (start 74.803 59.182) (end 74.803 66.675) (width 0.3) (layer "F.Cu") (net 4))
 (segment (start 62.295 54.229) (end 68.961 54.229) (width 0.3) (layer "F.Cu") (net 4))
 (segment (start 74.803 66.675) (end 73.787 67.691) (width 0.3) (layer "F.Cu") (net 4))
 (segment (start 61.025 55.499) (end 62.295 54.229) (width 0.3) (layer "F.Cu") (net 4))
 (segment (start 69.977 59.182) (end 74.803 59.182) (width 0.3) (layer "F.Cu") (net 4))
 (segment (start 73.787 74.168) (end 73.025 74.93) (width 0.3) (layer "F.Cu") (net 20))
 (segment (start 73.787 72.39) (end 73.787 74.168) (width 0.3) (layer "F.Cu") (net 20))
 (segment (start 67.35 83.272) (end 67.35 89.545) (width 0.3) (layer "F.Cu") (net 20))
 (segment (start 73.025 77.597) (end 67.35 83.272) (width 0.3) (layer "F.Cu") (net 20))
 (via (at 73.025 77.597) (size 0.7) (drill 0.3) (layers "F.Cu" "B.Cu") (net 20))
 (via (at 73.025 74.93) (size 0.7) (drill 0.3) (layers "F.Cu" "B.Cu") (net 20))
 (segment (start 73.025 74.93) (end 73.025 77.597) (width 0.3) (layer "B.Cu") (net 20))
 (segment (start 71.882 61.595) (end 55.372 61.595) (width 0.3) (layer "F.Cu") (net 11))
 (segment (start 73.406 63.119) (end 71.882 61.595) (width 0.3) (layer "F.Cu") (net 11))
 (segment (start 55.372 61.595) (end 53.848 63.119) (width 0.3) (layer "F.Cu") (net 11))
 (segment (start 50.8 48.26) (end 50.8 55.88) (width 0.5) (layer "F.Cu") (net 10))
 (segment (start 53.975 59.182) (end 53.987 59.17) (width 0.3) (layer "F.Cu") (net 9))
 (segment (start 53.594 59.182) (end 53.975 59.182) (width 0.3) (layer "F.Cu") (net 9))
 (segment (start 53.987 59.17) (end 55.433 59.17) (width 0.3) (layer "F.Cu") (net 9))
 (segment (start 53.594 48.514) (end 53.594 59.182) (width 0.3) (layer "F.Cu") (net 9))
 (segment (start 50.8 45.72) (end 53.594 48.514) (width 0.3) (layer "F.Cu") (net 9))
 (segment (start 75.692 75.819) (end 75.692 57.912) (width 0.3) (layer "F.Cu") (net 12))
 (segment (start 75.692 57.912) (end 73.66 55.88) (width 0.3) (layer "F.Cu") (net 12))
 (segment (start 50.802 75.44) (end 51.181 75.819) (width 0.3) (layer "F.Cu") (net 12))
 (segment (start 56.007 75.819) (end 75.692 75.819) (width 0.3) (layer "F.Cu") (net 12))
 (segment (start 73.66 45.72) (end 73.66 55.88) (width 0.5) (layer "F.Cu") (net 12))
 (segment (start 50.802 74.041) (end 50.802 75.44) (width 0.3) (layer "F.Cu") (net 12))
 (via (at 56.007 75.819) (size 0.7) (drill 0.3) (layers "F.Cu" "B.Cu") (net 12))
 (via (at 51.181 75.819) (size 0.7) (drill 0.3) (layers "F.Cu" "B.Cu") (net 12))
 (segment (start 51.181 75.819) (end 56.007 75.819) (width 0.3) (layer "B.Cu") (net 12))
 (segment (start 61.025 56.769) (end 60.608738 56.769) (width 0.3) (layer "F.Cu") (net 5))
 (segment (start 58.310738 54.471) (end 56.455 54.471) (width 0.3) (layer "F.Cu") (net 5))
 (segment (start 59.450869 55.611131) (end 58.310738 54.471) (width 0.3) (layer "F.Cu") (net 5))
 (segment (start 62.23 73.035) (end 62.23 62.484) (width 0.3) (layer "F.Cu") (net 5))
 (segment (start 60.608738 56.769) (end 59.450869 55.611131) (width 0.3) (layer "F.Cu") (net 5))
 (via (at 62.23 62.484) (size 0.7) (drill 0.3) (layers "F.Cu" "B.Cu") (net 5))
 (via (at 59.450869 55.611131) (size 0.7) (drill 0.3) (layers "F.Cu" "B.Cu") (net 5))
 (segment (start 59.450869 59.704869) (end 59.450869 55.611131) (width 0.3) (layer "B.Cu") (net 5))
 (segment (start 62.23 62.484) (end 59.450869 59.704869) (width 0.3) (layer "B.Cu") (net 5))
 (segment (start 49.782 70.622) (end 49.772 70.612) (width 0.3) (layer "F.Cu") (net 13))
 (segment (start 49.782 74.041) (end 49.782 70.622) (width 0.3) (layer "F.Cu") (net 13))
 (segment (start 51.042 70.612) (end 49.772 70.612) (width 0.3) (layer "F.Cu") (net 13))
 (segment (start 52.312 63.635) (end 52.828 63.119) (width 0.3) (layer "F.Cu") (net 19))
 (segment (start 52.312 65.662) (end 51.042 65.662) (width 0.3) (layer "F.Cu") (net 19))
 (segment (start 52.312 65.662) (end 52.312 63.635) (width 0.3) (layer "F.Cu") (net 19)))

